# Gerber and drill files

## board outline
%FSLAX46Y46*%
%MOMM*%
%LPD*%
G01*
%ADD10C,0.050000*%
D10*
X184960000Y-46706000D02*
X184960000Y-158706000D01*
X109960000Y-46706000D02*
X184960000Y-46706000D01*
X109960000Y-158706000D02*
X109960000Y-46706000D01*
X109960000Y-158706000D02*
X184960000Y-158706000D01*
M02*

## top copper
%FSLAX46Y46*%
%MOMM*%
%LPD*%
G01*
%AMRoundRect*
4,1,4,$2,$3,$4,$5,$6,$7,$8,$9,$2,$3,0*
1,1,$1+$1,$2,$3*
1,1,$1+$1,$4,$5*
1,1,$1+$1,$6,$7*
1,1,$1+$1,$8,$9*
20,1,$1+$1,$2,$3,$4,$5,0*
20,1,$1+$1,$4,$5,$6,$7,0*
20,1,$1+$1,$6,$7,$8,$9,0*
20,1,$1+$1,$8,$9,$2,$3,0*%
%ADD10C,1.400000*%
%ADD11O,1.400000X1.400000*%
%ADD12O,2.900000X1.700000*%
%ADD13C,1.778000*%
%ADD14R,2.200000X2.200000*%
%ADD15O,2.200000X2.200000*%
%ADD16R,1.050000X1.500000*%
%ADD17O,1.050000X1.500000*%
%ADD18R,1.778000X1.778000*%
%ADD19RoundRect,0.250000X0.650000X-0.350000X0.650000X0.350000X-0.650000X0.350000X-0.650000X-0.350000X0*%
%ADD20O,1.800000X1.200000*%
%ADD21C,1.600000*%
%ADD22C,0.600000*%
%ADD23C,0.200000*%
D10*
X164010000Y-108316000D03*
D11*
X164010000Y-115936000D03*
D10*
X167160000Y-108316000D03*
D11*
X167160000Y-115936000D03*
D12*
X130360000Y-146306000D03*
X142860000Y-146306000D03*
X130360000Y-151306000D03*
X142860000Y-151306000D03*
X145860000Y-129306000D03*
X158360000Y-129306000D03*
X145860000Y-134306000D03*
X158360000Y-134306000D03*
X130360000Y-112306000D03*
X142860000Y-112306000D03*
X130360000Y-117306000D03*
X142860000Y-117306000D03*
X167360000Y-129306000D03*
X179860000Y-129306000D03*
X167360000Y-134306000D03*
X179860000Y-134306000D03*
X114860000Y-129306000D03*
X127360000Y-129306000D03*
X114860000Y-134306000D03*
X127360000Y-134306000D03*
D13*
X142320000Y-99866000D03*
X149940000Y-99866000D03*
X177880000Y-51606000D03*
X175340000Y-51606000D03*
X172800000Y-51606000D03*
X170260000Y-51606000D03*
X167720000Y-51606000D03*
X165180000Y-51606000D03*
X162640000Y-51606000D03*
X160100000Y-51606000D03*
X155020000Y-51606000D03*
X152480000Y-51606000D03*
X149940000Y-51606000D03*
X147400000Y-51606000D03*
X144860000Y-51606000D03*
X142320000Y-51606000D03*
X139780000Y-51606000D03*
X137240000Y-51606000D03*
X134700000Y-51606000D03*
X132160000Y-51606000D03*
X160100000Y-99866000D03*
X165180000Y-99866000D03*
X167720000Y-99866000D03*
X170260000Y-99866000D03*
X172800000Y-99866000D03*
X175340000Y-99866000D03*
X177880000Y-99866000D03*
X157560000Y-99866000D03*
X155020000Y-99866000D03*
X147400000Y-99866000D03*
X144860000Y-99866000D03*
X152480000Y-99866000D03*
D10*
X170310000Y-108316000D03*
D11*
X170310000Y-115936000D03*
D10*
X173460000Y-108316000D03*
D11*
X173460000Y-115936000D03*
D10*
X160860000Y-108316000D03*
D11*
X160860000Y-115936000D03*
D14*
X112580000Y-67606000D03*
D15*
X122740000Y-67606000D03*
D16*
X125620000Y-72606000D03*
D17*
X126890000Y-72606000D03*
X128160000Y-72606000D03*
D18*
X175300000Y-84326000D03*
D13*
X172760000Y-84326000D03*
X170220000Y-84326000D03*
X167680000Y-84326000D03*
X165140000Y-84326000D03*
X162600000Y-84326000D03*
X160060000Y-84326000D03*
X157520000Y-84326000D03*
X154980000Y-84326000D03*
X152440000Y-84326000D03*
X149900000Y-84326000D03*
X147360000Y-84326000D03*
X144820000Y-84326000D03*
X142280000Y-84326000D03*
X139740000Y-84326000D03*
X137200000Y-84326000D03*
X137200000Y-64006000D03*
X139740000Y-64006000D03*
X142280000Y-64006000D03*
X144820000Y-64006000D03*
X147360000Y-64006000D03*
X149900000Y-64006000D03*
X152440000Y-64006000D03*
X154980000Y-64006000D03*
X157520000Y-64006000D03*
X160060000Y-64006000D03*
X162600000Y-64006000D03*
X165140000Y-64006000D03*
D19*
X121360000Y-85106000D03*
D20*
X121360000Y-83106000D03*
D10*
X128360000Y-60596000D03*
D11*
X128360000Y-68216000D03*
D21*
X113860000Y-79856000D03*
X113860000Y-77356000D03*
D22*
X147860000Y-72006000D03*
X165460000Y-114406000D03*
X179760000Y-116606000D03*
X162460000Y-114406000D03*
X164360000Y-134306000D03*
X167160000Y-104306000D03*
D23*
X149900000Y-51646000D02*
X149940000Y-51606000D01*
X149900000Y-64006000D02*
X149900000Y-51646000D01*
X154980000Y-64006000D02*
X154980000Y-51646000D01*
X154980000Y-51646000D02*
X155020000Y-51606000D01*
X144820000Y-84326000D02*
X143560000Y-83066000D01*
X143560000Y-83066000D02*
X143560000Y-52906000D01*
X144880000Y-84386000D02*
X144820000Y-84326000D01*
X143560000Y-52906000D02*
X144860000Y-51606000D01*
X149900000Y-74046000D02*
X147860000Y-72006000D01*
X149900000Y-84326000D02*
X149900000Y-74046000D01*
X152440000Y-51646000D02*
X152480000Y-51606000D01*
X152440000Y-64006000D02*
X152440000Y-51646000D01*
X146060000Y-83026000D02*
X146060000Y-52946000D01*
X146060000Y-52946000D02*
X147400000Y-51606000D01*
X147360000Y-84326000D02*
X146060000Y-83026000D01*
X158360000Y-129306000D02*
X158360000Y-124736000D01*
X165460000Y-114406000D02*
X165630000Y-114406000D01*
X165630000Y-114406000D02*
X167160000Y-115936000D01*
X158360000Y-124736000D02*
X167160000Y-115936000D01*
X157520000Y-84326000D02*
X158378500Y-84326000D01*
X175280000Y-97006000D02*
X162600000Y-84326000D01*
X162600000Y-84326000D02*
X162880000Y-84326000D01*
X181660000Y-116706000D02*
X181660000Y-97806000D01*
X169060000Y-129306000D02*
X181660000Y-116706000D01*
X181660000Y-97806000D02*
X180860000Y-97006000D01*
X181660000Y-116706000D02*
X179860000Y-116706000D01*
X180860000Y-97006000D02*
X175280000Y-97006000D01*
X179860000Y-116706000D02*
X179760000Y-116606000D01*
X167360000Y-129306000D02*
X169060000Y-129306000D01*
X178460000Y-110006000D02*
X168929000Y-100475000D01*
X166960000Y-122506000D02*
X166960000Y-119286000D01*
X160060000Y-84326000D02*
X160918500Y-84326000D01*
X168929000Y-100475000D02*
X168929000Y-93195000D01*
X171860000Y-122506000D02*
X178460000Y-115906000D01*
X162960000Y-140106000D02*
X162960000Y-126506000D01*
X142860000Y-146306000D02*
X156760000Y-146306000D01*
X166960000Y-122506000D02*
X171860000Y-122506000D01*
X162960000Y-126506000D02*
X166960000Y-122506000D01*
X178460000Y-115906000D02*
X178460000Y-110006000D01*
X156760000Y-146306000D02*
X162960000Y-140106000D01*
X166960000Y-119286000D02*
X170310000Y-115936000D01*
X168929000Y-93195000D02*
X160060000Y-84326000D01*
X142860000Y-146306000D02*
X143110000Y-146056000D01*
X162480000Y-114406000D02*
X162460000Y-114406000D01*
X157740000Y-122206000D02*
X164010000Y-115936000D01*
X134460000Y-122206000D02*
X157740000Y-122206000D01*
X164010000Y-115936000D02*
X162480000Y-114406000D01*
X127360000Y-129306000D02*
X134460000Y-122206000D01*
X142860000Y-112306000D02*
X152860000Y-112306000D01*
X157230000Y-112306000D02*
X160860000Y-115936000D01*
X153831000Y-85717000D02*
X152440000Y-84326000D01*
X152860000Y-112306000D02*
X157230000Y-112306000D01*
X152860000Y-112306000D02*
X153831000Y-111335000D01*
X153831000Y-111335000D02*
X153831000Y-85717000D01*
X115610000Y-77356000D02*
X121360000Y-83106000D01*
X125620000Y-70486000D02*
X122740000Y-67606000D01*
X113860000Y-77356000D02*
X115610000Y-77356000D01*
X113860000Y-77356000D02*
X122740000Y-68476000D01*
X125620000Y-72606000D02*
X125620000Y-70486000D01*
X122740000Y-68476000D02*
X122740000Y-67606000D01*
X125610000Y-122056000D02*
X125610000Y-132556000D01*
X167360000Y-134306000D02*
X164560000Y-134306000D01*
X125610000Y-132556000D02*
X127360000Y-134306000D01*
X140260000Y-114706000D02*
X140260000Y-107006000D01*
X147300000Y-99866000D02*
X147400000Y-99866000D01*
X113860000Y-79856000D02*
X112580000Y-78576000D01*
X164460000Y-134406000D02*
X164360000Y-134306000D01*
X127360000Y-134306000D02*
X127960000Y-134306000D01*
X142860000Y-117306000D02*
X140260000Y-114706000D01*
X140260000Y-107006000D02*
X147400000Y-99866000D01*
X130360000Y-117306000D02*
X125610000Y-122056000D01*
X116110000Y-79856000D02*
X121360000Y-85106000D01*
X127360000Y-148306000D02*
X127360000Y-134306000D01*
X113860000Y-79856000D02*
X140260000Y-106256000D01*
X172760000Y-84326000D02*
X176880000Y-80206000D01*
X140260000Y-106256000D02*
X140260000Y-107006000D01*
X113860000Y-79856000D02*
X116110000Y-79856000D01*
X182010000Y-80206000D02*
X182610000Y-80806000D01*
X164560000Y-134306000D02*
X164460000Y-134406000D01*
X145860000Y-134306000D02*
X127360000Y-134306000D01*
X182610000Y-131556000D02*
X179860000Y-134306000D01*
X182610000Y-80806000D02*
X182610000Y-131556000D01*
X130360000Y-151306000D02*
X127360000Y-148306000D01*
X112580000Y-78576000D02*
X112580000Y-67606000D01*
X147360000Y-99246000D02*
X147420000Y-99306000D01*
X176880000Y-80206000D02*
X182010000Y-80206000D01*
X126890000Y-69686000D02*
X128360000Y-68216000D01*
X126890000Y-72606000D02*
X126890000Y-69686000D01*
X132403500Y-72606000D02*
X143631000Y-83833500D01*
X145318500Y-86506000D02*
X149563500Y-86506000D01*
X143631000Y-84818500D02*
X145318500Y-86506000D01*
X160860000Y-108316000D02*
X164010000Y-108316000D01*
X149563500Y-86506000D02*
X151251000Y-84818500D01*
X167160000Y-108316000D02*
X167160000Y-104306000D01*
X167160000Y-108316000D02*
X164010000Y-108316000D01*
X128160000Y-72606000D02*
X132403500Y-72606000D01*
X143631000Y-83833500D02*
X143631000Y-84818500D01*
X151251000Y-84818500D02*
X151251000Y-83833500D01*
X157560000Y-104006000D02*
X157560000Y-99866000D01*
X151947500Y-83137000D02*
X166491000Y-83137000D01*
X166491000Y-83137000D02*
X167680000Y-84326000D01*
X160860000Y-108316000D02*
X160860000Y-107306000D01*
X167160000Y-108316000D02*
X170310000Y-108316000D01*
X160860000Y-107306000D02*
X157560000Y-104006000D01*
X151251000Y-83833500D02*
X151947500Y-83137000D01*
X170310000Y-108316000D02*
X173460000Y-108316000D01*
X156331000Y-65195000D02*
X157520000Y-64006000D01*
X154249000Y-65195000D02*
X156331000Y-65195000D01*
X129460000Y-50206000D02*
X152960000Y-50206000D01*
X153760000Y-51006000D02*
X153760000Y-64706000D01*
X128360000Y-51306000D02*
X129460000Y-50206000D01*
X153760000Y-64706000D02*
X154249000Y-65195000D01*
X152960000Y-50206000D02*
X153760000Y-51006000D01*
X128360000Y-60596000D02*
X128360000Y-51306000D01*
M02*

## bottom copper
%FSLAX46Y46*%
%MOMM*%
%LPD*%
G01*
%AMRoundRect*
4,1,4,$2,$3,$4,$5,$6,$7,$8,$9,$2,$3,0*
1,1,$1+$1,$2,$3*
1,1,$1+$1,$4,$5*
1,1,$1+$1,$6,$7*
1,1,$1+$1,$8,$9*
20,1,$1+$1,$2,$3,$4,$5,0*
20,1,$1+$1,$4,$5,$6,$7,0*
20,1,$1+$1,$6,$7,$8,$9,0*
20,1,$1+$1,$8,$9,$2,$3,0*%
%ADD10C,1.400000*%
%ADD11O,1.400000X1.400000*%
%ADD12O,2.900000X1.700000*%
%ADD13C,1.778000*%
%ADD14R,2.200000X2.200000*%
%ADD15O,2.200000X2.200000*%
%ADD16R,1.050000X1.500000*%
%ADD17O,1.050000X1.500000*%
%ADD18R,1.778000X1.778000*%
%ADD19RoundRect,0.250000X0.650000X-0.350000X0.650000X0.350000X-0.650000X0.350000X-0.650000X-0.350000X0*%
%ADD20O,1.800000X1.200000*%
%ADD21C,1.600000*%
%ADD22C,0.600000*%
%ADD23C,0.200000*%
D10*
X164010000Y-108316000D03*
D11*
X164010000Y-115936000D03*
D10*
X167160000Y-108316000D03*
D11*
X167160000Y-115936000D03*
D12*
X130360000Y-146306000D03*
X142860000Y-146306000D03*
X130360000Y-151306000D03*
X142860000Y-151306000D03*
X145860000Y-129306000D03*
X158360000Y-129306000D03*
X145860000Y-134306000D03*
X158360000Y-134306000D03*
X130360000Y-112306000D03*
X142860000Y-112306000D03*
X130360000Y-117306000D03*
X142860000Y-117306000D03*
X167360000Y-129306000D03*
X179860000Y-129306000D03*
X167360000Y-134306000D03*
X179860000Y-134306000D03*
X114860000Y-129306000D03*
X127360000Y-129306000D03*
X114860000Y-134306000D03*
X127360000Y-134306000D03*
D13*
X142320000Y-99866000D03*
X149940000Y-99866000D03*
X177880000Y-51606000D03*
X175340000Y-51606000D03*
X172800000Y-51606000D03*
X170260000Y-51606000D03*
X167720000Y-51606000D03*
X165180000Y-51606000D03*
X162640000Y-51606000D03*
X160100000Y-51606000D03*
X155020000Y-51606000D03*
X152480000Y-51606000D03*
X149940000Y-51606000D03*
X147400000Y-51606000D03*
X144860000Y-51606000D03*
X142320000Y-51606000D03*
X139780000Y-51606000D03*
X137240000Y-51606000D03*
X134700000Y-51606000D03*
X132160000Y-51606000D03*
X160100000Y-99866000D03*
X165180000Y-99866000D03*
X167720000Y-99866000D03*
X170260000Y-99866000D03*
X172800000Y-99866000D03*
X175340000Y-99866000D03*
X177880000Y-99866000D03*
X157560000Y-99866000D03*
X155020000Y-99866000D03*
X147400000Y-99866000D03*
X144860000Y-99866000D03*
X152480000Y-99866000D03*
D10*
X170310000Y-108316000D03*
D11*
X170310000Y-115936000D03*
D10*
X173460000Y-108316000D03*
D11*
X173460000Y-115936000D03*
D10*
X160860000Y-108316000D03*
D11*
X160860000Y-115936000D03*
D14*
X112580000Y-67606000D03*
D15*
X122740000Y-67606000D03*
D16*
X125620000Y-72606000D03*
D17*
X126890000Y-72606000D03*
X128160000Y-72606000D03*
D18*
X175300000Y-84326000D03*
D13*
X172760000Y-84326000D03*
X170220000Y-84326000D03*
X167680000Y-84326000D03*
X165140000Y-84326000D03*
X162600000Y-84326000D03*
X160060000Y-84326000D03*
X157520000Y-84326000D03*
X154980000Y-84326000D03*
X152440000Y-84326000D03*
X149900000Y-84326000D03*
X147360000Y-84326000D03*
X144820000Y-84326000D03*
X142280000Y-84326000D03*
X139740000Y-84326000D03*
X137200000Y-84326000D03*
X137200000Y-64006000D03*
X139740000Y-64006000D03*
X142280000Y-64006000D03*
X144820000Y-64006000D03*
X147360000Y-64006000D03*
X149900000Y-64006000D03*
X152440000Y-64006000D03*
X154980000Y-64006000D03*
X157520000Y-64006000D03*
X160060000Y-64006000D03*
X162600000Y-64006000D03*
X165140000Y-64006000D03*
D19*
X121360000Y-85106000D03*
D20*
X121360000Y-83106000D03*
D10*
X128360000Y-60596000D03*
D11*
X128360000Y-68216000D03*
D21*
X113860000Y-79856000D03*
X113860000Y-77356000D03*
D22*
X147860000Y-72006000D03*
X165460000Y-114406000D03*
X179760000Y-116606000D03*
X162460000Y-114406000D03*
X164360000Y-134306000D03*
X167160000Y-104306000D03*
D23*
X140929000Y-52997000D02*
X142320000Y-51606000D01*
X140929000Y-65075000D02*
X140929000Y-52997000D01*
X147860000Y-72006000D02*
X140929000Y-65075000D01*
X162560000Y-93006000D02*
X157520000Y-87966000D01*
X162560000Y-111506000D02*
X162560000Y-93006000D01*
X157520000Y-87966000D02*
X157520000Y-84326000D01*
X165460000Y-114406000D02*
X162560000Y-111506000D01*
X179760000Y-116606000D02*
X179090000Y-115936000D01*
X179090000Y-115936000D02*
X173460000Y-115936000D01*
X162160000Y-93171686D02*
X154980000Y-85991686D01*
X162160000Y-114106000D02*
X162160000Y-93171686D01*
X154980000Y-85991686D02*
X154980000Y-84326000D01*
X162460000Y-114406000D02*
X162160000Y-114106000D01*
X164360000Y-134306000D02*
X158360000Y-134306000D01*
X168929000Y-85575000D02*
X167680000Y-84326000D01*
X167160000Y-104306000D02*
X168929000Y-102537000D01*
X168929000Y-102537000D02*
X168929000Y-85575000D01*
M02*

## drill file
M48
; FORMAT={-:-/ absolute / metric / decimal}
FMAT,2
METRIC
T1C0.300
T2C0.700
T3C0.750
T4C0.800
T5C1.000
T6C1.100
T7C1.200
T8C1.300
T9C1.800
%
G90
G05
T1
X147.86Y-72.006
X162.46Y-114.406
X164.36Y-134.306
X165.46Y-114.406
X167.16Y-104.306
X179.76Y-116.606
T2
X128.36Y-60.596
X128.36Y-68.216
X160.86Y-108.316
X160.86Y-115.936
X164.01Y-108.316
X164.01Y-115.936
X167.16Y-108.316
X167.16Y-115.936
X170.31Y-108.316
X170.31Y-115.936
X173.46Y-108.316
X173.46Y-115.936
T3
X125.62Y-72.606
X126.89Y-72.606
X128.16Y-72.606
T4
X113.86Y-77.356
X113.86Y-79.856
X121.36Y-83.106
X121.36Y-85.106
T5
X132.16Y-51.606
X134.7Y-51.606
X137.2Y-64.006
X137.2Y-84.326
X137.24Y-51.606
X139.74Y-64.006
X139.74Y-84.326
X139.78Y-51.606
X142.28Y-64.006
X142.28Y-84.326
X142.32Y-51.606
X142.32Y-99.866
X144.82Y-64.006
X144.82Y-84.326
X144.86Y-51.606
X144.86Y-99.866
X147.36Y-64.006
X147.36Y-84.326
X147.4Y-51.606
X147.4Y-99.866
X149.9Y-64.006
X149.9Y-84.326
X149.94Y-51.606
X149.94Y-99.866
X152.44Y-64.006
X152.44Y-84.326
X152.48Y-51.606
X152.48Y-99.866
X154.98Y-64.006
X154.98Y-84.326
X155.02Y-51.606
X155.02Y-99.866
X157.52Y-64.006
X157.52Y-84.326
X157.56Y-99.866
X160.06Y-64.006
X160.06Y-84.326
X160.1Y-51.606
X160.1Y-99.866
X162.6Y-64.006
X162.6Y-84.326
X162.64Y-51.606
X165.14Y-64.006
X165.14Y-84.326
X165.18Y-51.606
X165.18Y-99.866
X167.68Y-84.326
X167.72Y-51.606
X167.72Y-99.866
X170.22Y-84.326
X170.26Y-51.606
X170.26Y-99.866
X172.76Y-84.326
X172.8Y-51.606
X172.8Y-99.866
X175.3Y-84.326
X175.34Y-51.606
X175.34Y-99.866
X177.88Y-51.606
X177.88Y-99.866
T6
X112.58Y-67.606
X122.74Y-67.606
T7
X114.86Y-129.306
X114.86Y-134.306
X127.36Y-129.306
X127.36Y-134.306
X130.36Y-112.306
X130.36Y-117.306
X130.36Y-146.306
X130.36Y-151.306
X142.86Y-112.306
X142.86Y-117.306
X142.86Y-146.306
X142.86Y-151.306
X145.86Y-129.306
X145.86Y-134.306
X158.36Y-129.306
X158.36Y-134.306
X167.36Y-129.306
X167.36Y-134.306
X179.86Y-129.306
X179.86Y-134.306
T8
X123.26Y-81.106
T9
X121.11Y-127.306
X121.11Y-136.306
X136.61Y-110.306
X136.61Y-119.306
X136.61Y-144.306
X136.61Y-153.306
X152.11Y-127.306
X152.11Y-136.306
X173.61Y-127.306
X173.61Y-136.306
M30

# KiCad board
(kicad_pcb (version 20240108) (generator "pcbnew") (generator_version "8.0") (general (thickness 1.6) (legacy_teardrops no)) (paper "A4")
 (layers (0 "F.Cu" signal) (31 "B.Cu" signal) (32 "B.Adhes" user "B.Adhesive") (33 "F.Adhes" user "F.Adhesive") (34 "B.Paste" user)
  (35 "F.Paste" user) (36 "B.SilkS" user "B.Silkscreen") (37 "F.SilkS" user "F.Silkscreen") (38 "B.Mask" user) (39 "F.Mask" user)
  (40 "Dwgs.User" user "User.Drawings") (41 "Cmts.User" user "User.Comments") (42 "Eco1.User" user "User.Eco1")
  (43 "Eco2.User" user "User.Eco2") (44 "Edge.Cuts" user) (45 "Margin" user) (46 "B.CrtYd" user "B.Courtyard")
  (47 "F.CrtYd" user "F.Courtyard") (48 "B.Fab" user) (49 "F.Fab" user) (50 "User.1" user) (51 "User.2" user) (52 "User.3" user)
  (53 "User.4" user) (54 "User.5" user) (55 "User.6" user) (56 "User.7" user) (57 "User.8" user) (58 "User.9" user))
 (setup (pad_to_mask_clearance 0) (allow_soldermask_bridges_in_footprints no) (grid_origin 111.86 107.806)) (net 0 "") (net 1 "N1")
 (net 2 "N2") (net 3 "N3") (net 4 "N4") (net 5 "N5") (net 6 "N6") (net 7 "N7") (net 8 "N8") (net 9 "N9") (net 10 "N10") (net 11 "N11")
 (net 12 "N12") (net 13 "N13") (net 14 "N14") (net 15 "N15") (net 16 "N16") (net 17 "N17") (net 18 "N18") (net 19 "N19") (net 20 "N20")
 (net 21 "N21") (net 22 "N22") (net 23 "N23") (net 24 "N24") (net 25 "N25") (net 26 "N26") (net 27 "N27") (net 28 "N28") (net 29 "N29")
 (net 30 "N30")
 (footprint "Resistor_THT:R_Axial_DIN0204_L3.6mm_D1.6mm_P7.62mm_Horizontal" (layer "F.Cu") (at 164.01 108.316 -90)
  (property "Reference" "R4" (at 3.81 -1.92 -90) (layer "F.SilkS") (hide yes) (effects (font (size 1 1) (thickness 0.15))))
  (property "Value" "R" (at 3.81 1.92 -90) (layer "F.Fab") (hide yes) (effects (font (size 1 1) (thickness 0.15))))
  (pad "1" thru_hole circle (at 0 0 270) (size 1.4 1.4) (drill 0.7) (layers "*.Cu" "*.Mask") (remove_unused_layers no) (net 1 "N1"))
  (pad "2" thru_hole oval (at 7.62 0 270) (size 1.4 1.4) (drill 0.7) (layers "*.Cu" "*.Mask") (remove_unused_layers no) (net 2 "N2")))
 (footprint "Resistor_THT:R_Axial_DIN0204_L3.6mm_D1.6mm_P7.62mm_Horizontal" (layer "F.Cu") (at 167.16 108.316 -90)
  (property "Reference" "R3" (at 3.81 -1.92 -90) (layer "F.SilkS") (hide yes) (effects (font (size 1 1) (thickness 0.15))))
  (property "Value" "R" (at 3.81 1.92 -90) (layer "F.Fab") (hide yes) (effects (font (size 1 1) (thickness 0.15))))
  (pad "1" thru_hole circle (at 0 0 270) (size 1.4 1.4) (drill 0.7) (layers "*.Cu" "*.Mask") (remove_unused_layers no) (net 1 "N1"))
  (pad "2" thru_hole oval (at 7.62 0 270) (size 1.4 1.4) (drill 0.7) (layers "*.Cu" "*.Mask") (remove_unused_layers no) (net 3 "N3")))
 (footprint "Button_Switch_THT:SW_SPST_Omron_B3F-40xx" (layer "F.Cu") (at 130.36 146.306)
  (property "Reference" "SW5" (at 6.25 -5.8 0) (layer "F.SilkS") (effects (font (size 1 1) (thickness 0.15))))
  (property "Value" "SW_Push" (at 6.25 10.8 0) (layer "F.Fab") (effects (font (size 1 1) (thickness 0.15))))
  (pad "" np_thru_hole circle (at 6.25 -2) (size 1.8 1.8) (drill 1.8) (layers "F&B.Cu" "*.Mask"))
  (pad "" np_thru_hole circle (at 6.25 7) (size 1.8 1.8) (drill 1.8) (layers "F&B.Cu" "*.Mask"))
  (pad "1" thru_hole oval (at 0 0) (size 2.9 1.7) (drill 1.2) (layers "*.Cu" "*.Mask") (remove_unused_layers no) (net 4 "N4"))
  (pad "1" thru_hole oval (at 12.5 0) (size 2.9 1.7) (drill 1.2) (layers "*.Cu" "*.Mask") (remove_unused_layers no) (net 4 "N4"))
  (pad "2" thru_hole oval (at 0 5) (size 2.9 1.7) (drill 1.2) (layers "*.Cu" "*.Mask") (remove_unused_layers no) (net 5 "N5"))
  (pad "2" thru_hole oval (at 12.5 5) (size 2.9 1.7) (drill 1.2) (layers "*.Cu" "*.Mask") (remove_unused_layers no) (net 5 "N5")))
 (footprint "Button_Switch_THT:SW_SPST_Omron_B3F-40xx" (layer "F.Cu") (at 145.86 129.306)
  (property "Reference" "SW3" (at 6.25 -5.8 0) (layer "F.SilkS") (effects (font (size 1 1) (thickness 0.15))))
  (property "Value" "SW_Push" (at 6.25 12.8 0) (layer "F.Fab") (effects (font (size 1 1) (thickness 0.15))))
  (pad "" np_thru_hole circle (at 6.25 -2) (size 1.8 1.8) (drill 1.8) (layers "F&B.Cu" "*.Mask"))
  (pad "" np_thru_hole circle (at 6.25 7) (size 1.8 1.8) (drill 1.8) (layers "F&B.Cu" "*.Mask"))
  (pad "1" thru_hole oval (at 0 0) (size 2.9 1.7) (drill 1.2) (layers "*.Cu" "*.Mask") (remove_unused_layers no) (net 3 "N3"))
  (pad "1" thru_hole oval (at 12.5 0) (size 2.9 1.7) (drill 1.2) (layers "*.Cu" "*.Mask") (remove_unused_layers no) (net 3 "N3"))
  (pad "2" thru_hole oval (at 0 5) (size 2.9 1.7) (drill 1.2) (layers "*.Cu" "*.Mask") (remove_unused_layers no) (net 5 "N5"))
  (pad "2" thru_hole oval (at 12.5 5) (size 2.9 1.7) (drill 1.2) (layers "*.Cu" "*.Mask") (remove_unused_layers no) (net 5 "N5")))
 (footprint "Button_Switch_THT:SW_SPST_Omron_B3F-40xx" (layer "F.Cu") (at 130.36 112.306)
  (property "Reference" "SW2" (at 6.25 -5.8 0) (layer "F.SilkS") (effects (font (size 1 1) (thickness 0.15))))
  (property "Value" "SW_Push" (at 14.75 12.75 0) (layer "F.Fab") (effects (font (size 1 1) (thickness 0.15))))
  (pad "" np_thru_hole circle (at 6.25 -2) (size 1.8 1.8) (drill 1.8) (layers "F&B.Cu" "*.Mask"))
  (pad "" np_thru_hole circle (at 6.25 7) (size 1.8 1.8) (drill 1.8) (layers "F&B.Cu" "*.Mask"))
  (pad "1" thru_hole oval (at 0 0) (size 2.9 1.7) (drill 1.2) (layers "*.Cu" "*.Mask") (remove_unused_layers no) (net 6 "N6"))
  (pad "1" thru_hole oval (at 12.5 0) (size 2.9 1.7) (drill 1.2) (layers "*.Cu" "*.Mask") (remove_unused_layers no) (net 6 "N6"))
  (pad "2" thru_hole oval (at 0 5) (size 2.9 1.7) (drill 1.2) (layers "*.Cu" "*.Mask") (remove_unused_layers no) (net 5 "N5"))
  (pad "2" thru_hole oval (at 12.5 5) (size 2.9 1.7) (drill 1.2) (layers "*.Cu" "*.Mask") (remove_unused_layers no) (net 5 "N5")))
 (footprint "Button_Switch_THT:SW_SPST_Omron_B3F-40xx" (layer "F.Cu") (at 167.36 129.306)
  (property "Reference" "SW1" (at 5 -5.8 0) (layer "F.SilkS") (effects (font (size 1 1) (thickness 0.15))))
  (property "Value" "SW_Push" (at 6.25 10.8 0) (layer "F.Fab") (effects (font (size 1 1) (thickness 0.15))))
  (pad "" np_thru_hole circle (at 6.25 -2) (size 1.8 1.8) (drill 1.8) (layers "F&B.Cu" "*.Mask"))
  (pad "" np_thru_hole circle (at 6.25 7) (size 1.8 1.8) (drill 1.8) (layers "F&B.Cu" "*.Mask"))
  (pad "1" thru_hole oval (at 0 0) (size 2.9 1.7) (drill 1.2) (layers "*.Cu" "*.Mask") (remove_unused_layers no) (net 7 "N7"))
  (pad "1" thru_hole oval (at 12.5 0) (size 2.9 1.7) (drill 1.2) (layers "*.Cu" "*.Mask") (remove_unused_layers no) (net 7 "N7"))
  (pad "2" thru_hole oval (at 0 5) (size 2.9 1.7) (drill 1.2) (layers "*.Cu" "*.Mask") (remove_unused_layers no) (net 5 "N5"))
  (pad "2" thru_hole oval (at 12.5 5) (size 2.9 1.7) (drill 1.2) (layers "*.Cu" "*.Mask") (remove_unused_layers no) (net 5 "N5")))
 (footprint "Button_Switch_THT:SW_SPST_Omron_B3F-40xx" (layer "F.Cu") (at 114.86 129.306)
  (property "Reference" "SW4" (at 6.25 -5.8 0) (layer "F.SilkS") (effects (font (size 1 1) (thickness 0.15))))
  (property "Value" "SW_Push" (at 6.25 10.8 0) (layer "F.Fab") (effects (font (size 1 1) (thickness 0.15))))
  (pad "" np_thru_hole circle (at 6.25 -2) (size 1.8 1.8) (drill 1.8) (layers "F&B.Cu" "*.Mask"))
  (pad "" np_thru_hole circle (at 6.25 7) (size 1.8 1.8) (drill 1.8) (layers "F&B.Cu" "*.Mask"))
  (pad "1" thru_hole oval (at 0 0) (size 2.9 1.7) (drill 1.2) (layers "*.Cu" "*.Mask") (remove_unused_layers no) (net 2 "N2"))
  (pad "1" thru_hole oval (at 12.5 0) (size 2.9 1.7) (drill 1.2) (layers "*.Cu" "*.Mask") (remove_unused_layers no) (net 2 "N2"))
  (pad "2" thru_hole oval (at 0 5) (size 2.9 1.7) (drill 1.2) (layers "*.Cu" "*.Mask") (remove_unused_layers no) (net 5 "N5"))
  (pad "2" thru_hole oval (at 12.5 5) (size 2.9 1.7) (drill 1.2) (layers "*.Cu" "*.Mask") (remove_unused_layers no) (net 5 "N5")))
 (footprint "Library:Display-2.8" (layer "F.Cu") (at 177.88 51.606 90)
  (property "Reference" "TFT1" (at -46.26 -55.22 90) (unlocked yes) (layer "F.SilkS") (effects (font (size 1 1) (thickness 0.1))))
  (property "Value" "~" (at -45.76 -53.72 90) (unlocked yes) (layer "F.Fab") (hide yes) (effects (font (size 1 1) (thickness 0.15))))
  (pad "" thru_hole circle (at -48.26 -35.56 90) (size 1.778 1.778) (drill 1) (layers "*.Cu" "*.Mask") (remove_unused_layers no))
  (pad "" thru_hole circle (at -48.26 -27.94 90) (size 1.778 1.778) (drill 1) (layers "*.Cu" "*.Mask") (remove_unused_layers no))
  (pad "0" thru_hole circle (at 0 0 90) (size 1.778 1.778) (drill 1) (layers "*.Cu" "*.Mask") (remove_unused_layers no))
  (pad "1" thru_hole circle (at 0 -2.54 90) (size 1.778 1.778) (drill 1) (layers "*.Cu" "*.Mask") (remove_unused_layers no))
  (pad "2" thru_hole circle (at 0 -5.08 90) (size 1.778 1.778) (drill 1) (layers "*.Cu" "*.Mask") (remove_unused_layers no))
  (pad "3" thru_hole circle (at 0 -7.62 90) (size 1.778 1.778) (drill 1) (layers "*.Cu" "*.Mask") (remove_unused_layers no))
  (pad "4" thru_hole circle (at 0 -10.16 90) (size 1.778 1.778) (drill 1) (layers "*.Cu" "*.Mask") (remove_unused_layers no) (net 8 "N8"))
  (pad "5" thru_hole circle (at 0 -12.7 90) (size 1.778 1.778) (drill 1) (layers "*.Cu" "*.Mask") (remove_unused_layers no))
  (pad "6" thru_hole circle (at 0 -15.24 90) (size 1.778 1.778) (drill 1) (layers "*.Cu" "*.Mask") (remove_unused_layers no))
  (pad "7" thru_hole circle (at 0 -17.78 90) (size 1.778 1.778) (drill 1) (layers "*.Cu" "*.Mask") (remove_unused_layers no))
  (pad "8" thru_hole circle (at 0 -22.86 90) (size 1.778 1.778) (drill 1) (layers "*.Cu" "*.Mask") (remove_unused_layers no) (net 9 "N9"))
  (pad "9" thru_hole circle (at 0 -25.4 90) (size 1.778 1.778) (drill 1) (layers "*.Cu" "*.Mask") (remove_unused_layers no) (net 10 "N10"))
  (pad "10" thru_hole circle (at 0 -27.94 90) (size 1.778 1.778) (drill 1) (layers "*.Cu" "*.Mask") (remove_unused_layers no) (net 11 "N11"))
  (pad "11" thru_hole circle (at 0 -30.48 90) (size 1.778 1.778) (drill 1) (layers "*.Cu" "*.Mask") (remove_unused_layers no) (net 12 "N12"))
  (pad "12" thru_hole circle (at 0 -33.02 90) (size 1.778 1.778) (drill 1) (layers "*.Cu" "*.Mask") (remove_unused_layers no) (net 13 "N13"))
  (pad "13" thru_hole circle (at 0 -35.56 90) (size 1.778 1.778) (drill 1) (layers "*.Cu" "*.Mask" "Dwgs.User") (remove_unused_layers no)
   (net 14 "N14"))
  (pad "14" thru_hole circle (at 0 -38.1 90) (size 1.778 1.778) (drill 1) (layers "*.Cu" "B.Mask") (remove_unused_layers no))
  (pad "15" thru_hole circle (at 0 -40.64 90) (size 1.778 1.778) (drill 1) (layers "*.Cu" "*.Mask" "B.SilkS") (remove_unused_layers no))
  (pad "16" thru_hole circle (at 0 -43.18 90) (size 1.778 1.778) (drill 1) (layers "*.Cu" "*.Mask") (remove_unused_layers no))
  (pad "17" thru_hole circle (at 0 -45.72 90) (size 1.778 1.778) (drill 1) (layers "*.Cu" "*.Mask" "F.Paste") (remove_unused_layers no))
  (pad "22" thru_hole circle (at -48.26 -17.78 90) (size 1.778 1.778) (drill 1) (layers "*.Cu" "*.Mask") (remove_unused_layers no))
  (pad "23" thru_hole circle (at -48.26 -12.7 90) (size 1.778 1.778) (drill 1) (layers "*.Cu" "*.Mask") (remove_unused_layers no))
  (pad "24" thru_hole circle (at -48.26 -10.16 90) (size 1.778 1.778) (drill 1) (layers "*.Cu" "*.Mask") (remove_unused_layers no))
  (pad "25" thru_hole circle (at -48.26 -7.62 90) (size 1.778 1.778) (drill 1) (layers "*.Cu" "*.Mask") (remove_unused_layers no))
  (pad "26" thru_hole circle (at -48.26 -5.08 90) (size 1.778 1.778) (drill 1) (layers "*.Cu" "*.Mask") (remove_unused_layers no))
  (pad "27" thru_hole circle (at -48.26 -2.54 90) (size 1.778 1.778) (drill 1) (layers "*.Cu" "*.Mask") (remove_unused_layers no))
  (pad "28" thru_hole circle (at -48.26 0 90) (size 1.778 1.778) (drill 1) (layers "*.Cu" "*.Mask") (remove_unused_layers no))
  (pad "40" thru_hole circle (at -48.26 -20.32 90) (size 1.778 1.778) (drill 1) (layers "*.Cu" "*.Mask") (remove_unused_layers no)
   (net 1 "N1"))
  (pad "41" thru_hole circle (at -48.26 -22.86 90) (size 1.778 1.778) (drill 1) (layers "*.Cu" "*.Mask") (remove_unused_layers no))
  (pad "50" thru_hole circle (at -48.26 -30.48 90) (size 1.778 1.778) (drill 1) (layers "*.Cu" "*.Mask") (remove_unused_layers no)
   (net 5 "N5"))
  (pad "51" thru_hole circle (at -48.26 -33.02 90) (size 1.778 1.778) (drill 1) (layers "*.Cu" "*.Mask") (remove_unused_layers no))
  (pad "67" thru_hole circle (at -48.26 -25.4 90) (size 1.778 1.778) (drill 1) (layers "*.Cu" "*.Mask") (remove_unused_layers no)))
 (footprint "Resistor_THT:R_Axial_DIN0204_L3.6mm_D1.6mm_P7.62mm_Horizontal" (layer "F.Cu") (at 170.31 108.316 -90)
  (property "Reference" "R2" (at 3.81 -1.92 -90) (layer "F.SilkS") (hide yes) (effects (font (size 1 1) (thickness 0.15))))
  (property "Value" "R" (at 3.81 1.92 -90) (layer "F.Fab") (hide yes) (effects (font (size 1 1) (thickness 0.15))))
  (pad "1" thru_hole circle (at 0 0 270) (size 1.4 1.4) (drill 0.7) (layers "*.Cu" "*.Mask") (remove_unused_layers no) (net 1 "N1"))
  (pad "2" thru_hole oval (at 7.62 0 270) (size 1.4 1.4) (drill 0.7) (layers "*.Cu" "*.Mask") (remove_unused_layers no) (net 4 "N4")))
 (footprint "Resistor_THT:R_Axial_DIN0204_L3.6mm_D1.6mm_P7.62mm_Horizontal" (layer "F.Cu") (at 173.46 108.316 -90)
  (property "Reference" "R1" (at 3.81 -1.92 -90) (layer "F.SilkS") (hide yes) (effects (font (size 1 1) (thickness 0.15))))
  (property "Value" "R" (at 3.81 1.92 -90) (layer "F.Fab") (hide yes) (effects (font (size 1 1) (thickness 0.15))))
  (pad "1" thru_hole circle (at 0 0 270) (size 1.4 1.4) (drill 0.7) (layers "*.Cu" "*.Mask") (remove_unused_layers no) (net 1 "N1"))
  (pad "2" thru_hole oval (at 7.62 0 270) (size 1.4 1.4) (drill 0.7) (layers "*.Cu" "*.Mask") (remove_unused_layers no) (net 7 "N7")))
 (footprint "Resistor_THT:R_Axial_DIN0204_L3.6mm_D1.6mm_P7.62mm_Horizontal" (layer "F.Cu") (at 160.86 108.316 -90)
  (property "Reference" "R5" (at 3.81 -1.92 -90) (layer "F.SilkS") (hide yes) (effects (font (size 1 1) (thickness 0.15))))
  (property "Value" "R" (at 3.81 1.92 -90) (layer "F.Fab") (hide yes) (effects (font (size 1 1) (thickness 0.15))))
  (pad "1" thru_hole circle (at 0 0 270) (size 1.4 1.4) (drill 0.7) (layers "*.Cu" "*.Mask") (remove_unused_layers no) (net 1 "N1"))
  (pad "2" thru_hole oval (at 7.62 0 270) (size 1.4 1.4) (drill 0.7) (layers "*.Cu" "*.Mask") (remove_unused_layers no) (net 6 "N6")))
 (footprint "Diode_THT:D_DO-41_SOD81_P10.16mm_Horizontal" (layer "B.Cu") (at 112.58 67.606)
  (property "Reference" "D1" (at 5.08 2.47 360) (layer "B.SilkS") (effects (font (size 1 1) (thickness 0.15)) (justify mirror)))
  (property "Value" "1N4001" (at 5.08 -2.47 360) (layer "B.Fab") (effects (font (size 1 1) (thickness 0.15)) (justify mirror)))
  (pad "1" thru_hole rect (at 0 0) (size 2.2 2.2) (drill 1.1) (layers "*.Cu" "*.Mask") (remove_unused_layers no) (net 5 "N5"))
  (pad "2" thru_hole oval (at 10.16 0) (size 2.2 2.2) (drill 1.1) (layers "*.Cu" "*.Mask") (remove_unused_layers no) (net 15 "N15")))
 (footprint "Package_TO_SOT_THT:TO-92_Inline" (layer "B.Cu") (at 125.62 72.606)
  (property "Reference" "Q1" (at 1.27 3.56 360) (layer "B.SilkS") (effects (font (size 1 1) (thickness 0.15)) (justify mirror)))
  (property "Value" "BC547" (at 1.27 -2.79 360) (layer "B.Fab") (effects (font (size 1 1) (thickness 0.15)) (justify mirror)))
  (pad "1" thru_hole rect (at 0 0) (size 1.05 1.5) (drill 0.75) (layers "*.Cu" "*.Mask") (remove_unused_layers no) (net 15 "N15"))
  (pad "2" thru_hole oval (at 1.27 0) (size 1.05 1.5) (drill 0.75) (layers "*.Cu" "*.Mask") (remove_unused_layers no) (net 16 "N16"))
  (pad "3" thru_hole oval (at 2.54 0) (size 1.05 1.5) (drill 0.75) (layers "*.Cu" "*.Mask") (remove_unused_layers no) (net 1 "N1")))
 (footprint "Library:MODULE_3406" (layer "B.Cu") (at 156.25 74.166 90)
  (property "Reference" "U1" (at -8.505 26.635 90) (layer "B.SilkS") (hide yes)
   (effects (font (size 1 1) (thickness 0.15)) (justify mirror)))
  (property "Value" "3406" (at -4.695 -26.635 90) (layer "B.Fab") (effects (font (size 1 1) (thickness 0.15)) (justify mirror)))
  (pad "1" thru_hole rect (at -10.16 19.05 90) (size 1.778 1.778) (drill 1) (layers "*.Cu" "*.Mask") (remove_unused_layers no)
   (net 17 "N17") (solder_mask_margin 0.102))
  (pad "2" thru_hole circle (at -10.16 16.51 90) (size 1.778 1.778) (drill 1) (layers "*.Cu" "*.Mask") (remove_unused_layers no)
   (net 5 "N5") (solder_mask_margin 0.102))
  (pad "3" thru_hole circle (at -10.16 13.97 90) (size 1.778 1.778) (drill 1) (layers "*.Cu" "*.Mask") (remove_unused_layers no)
   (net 5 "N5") (solder_mask_margin 0.102))
  (pad "4" thru_hole circle (at -10.16 11.43 90) (size 1.778 1.778) (drill 1) (layers "*.Cu" "*.Mask") (remove_unused_layers no)
   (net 1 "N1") (solder_mask_margin 0.102))
  (pad "5" thru_hole circle (at -10.16 8.89 90) (size 1.778 1.778) (drill 1) (layers "*.Cu" "*.Mask") (remove_unused_layers no)
   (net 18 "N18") (solder_mask_margin 0.102))
  (pad "6" thru_hole circle (at -10.16 6.35 90) (size 1.778 1.778) (drill 1) (layers "*.Cu" "*.Mask") (remove_unused_layers no) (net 7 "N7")
   (solder_mask_margin 0.102))
  (pad "7" thru_hole circle (at -10.16 3.81 90) (size 1.778 1.778) (drill 1) (layers "*.Cu" "*.Mask") (remove_unused_layers no) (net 4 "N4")
   (solder_mask_margin 0.102))
  (pad "8" thru_hole circle (at -10.16 1.27 90) (size 1.778 1.778) (drill 1) (layers "*.Cu" "*.Mask") (remove_unused_layers no) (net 3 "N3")
   (solder_mask_margin 0.102))
  (pad "9" thru_hole circle (at -10.16 -1.27 90) (size 1.778 1.778) (drill 1) (layers "*.Cu" "*.Mask") (remove_unused_layers no)
   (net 2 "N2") (solder_mask_margin 0.102))
  (pad "10" thru_hole circle (at -10.16 -3.81 90) (size 1.778 1.778) (drill 1) (layers "*.Cu" "*.Mask") (remove_unused_layers no)
   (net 6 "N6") (solder_mask_margin 0.102))
  (pad "11" thru_hole circle (at -10.16 -6.35 90) (size 1.778 1.778) (drill 1) (layers "*.Cu" "*.Mask") (remove_unused_layers no)
   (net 14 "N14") (solder_mask_margin 0.102))
  (pad "12" thru_hole circle (at -10.16 -8.89 90) (size 1.778 1.778) (drill 1) (layers "*.Cu" "*.Mask") (remove_unused_layers no)
   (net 12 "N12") (solder_mask_margin 0.102))
  (pad "13" thru_hole circle (at -10.16 -11.43 90) (size 1.778 1.778) (drill 1) (layers "*.Cu" "*.Mask") (remove_unused_layers no)
   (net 13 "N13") (solder_mask_margin 0.102))
  (pad "14" thru_hole circle (at -10.16 -13.97 90) (size 1.778 1.778) (drill 1) (layers "*.Cu" "*.Mask") (remove_unused_layers no)
   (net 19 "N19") (solder_mask_margin 0.102))
  (pad "15" thru_hole circle (at -10.16 -16.51 90) (size 1.778 1.778) (drill 1) (layers "*.Cu" "*.Mask") (remove_unused_layers no)
   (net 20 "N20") (solder_mask_margin 0.102))
  (pad "16" thru_hole circle (at -10.16 -19.05 90) (size 1.778 1.778) (drill 1) (layers "*.Cu" "*.Mask") (remove_unused_layers no)
   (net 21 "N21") (solder_mask_margin 0.102))
  (pad "17" thru_hole circle (at 10.16 -19.05 90) (size 1.778 1.778) (drill 1) (layers "*.Cu" "*.Mask") (remove_unused_layers no)
   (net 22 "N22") (solder_mask_margin 0.102))
  (pad "18" thru_hole circle (at 10.16 -16.51 90) (size 1.778 1.778) (drill 1) (layers "*.Cu" "*.Mask") (remove_unused_layers no)
   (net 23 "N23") (solder_mask_margin 0.102))
  (pad "19" thru_hole circle (at 10.16 -13.97 90) (size 1.778 1.778) (drill 1) (layers "*.Cu" "*.Mask") (remove_unused_layers no)
   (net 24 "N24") (solder_mask_margin 0.102))
  (pad "20" thru_hole circle (at 10.16 -11.43 90) (size 1.778 1.778) (drill 1) (layers "*.Cu" "*.Mask") (remove_unused_layers no)
   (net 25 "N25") (solder_mask_margin 0.102))
  (pad "21" thru_hole circle (at 10.16 -8.89 90) (size 1.778 1.778) (drill 1) (layers "*.Cu" "*.Mask") (remove_unused_layers no)
   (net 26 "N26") (solder_mask_margin 0.102))
  (pad "22" thru_hole circle (at 10.16 -6.35 90) (size 1.778 1.778) (drill 1) (layers "*.Cu" "*.Mask") (remove_unused_layers no)
   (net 11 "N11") (solder_mask_margin 0.102))
  (pad "23" thru_hole circle (at 10.16 -3.81 90) (size 1.778 1.778) (drill 1) (layers "*.Cu" "*.Mask") (remove_unused_layers no)
   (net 10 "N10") (solder_mask_margin 0.102))
  (pad "24" thru_hole circle (at 10.16 -1.27 90) (size 1.778 1.778) (drill 1) (layers "*.Cu" "*.Mask") (remove_unused_layers no)
   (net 9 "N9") (solder_mask_margin 0.102))
  (pad "25" thru_hole circle (at 10.16 1.27 90) (size 1.778 1.778) (drill 1) (layers "*.Cu" "*.Mask") (remove_unused_layers no)
   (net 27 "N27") (solder_mask_margin 0.102))
  (pad "26" thru_hole circle (at 10.16 3.81 90) (size 1.778 1.778) (drill 1) (layers "*.Cu" "*.Mask") (remove_unused_layers no)
   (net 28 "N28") (solder_mask_margin 0.102))
  (pad "27" thru_hole circle (at 10.16 6.35 90) (size 1.778 1.778) (drill 1) (layers "*.Cu" "*.Mask") (remove_unused_layers no)
   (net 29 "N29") (solder_mask_margin 0.102))
  (pad "28" thru_hole circle (at 10.16 8.89 90) (size 1.778 1.778) (drill 1) (layers "*.Cu" "*.Mask") (remove_unused_layers no)
   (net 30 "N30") (solder_mask_margin 0.102)))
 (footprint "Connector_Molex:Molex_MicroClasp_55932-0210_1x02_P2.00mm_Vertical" (layer "B.Cu") (at 121.36 85.106 90)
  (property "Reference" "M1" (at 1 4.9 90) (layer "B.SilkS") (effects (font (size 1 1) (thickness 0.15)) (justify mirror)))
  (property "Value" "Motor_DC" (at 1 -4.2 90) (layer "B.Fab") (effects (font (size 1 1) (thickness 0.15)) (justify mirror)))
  (pad "" np_thru_hole circle (at 4 1.9 90) (size 1.3 1.3) (drill 1.3) (layers "*.Cu" "*.Mask"))
  (pad "1" thru_hole roundrect (at 0 0 90) (size 1.2 1.8) (drill 0.8) (layers "*.Cu" "*.Mask") (remove_unused_layers no)
   (roundrect_rratio 0.208333) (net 5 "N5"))
  (pad "2" thru_hole oval (at 2 0 90) (size 1.2 1.8) (drill 0.8) (layers "*.Cu" "*.Mask") (remove_unused_layers no) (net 15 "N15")))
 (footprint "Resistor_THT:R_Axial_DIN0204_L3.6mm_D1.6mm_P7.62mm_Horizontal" (layer "B.Cu") (at 128.36 60.596 -90)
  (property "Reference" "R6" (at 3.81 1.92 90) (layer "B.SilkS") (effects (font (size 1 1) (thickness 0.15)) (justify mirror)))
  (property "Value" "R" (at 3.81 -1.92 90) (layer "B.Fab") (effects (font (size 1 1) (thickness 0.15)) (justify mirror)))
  (pad "1" thru_hole circle (at 0 0 270) (size 1.4 1.4) (drill 0.7) (layers "*.Cu" "*.Mask") (remove_unused_layers no) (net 27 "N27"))
  (pad "2" thru_hole oval (at 7.62 0 270) (size 1.4 1.4) (drill 0.7) (layers "*.Cu" "*.Mask") (remove_unused_layers no) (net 16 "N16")))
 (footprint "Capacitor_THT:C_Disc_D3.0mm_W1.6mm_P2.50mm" (layer "B.Cu") (at 113.86 79.856 90)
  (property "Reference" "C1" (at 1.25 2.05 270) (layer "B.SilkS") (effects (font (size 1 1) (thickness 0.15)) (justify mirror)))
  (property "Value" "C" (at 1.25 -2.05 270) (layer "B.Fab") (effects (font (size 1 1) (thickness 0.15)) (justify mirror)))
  (pad "1" thru_hole circle (at 0 0 90) (size 1.6 1.6) (drill 0.8) (layers "*.Cu" "*.Mask") (remove_unused_layers no) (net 5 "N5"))
  (pad "2" thru_hole circle (at 2.5 0 90) (size 1.6 1.6) (drill 0.8) (layers "*.Cu" "*.Mask") (remove_unused_layers no) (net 15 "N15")))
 (gr_line (start 184.96 46.706) (end 184.96 158.706) (stroke (width 0.05) (type default)) (layer "Edge.Cuts"))
 (gr_line (start 109.96 46.706) (end 184.96 46.706) (stroke (width 0.05) (type default)) (layer "Edge.Cuts"))
 (gr_line (start 109.96 158.706) (end 109.96 46.706) (stroke (width 0.05) (type default)) (layer "Edge.Cuts"))
 (gr_line (start 109.96 158.706) (end 184.96 158.706) (stroke (width 0.05) (type default)) (layer "Edge.Cuts"))
 (segment (start 149.9 51.646) (end 149.94 51.606) (width 0.2) (layer "F.Cu") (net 11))
 (segment (start 149.9 64.006) (end 149.9 51.646) (width 0.2) (layer "F.Cu") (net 11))
 (segment (start 154.98 64.006) (end 154.98 51.646) (width 0.2) (layer "F.Cu") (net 9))
 (segment (start 154.98 51.646) (end 155.02 51.606) (width 0.2) (layer "F.Cu") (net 9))
 (segment (start 144.82 84.326) (end 143.56 83.066) (width 0.2) (layer "F.Cu") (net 13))
 (segment (start 143.56 83.066) (end 143.56 52.906) (width 0.2) (layer "F.Cu") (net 13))
 (segment (start 144.88 84.386) (end 144.82 84.326) (width 0.2) (layer "F.Cu") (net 13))
 (segment (start 143.56 52.906) (end 144.86 51.606) (width 0.2) (layer "F.Cu") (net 13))
 (segment (start 149.9 74.046) (end 147.86 72.006) (width 0.2) (layer "F.Cu") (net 14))
 (segment (start 149.9 84.326) (end 149.9 74.046) (width 0.2) (layer "F.Cu") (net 14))
 (via (at 147.86 72.006) (size 0.6) (drill 0.3) (layers "F.Cu" "B.Cu") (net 14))
 (segment (start 140.929 52.997) (end 142.32 51.606) (width 0.2) (layer "B.Cu") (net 14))
 (segment (start 140.929 65.075) (end 140.929 52.997) (width 0.2) (layer "B.Cu") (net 14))
 (segment (start 147.86 72.006) (end 140.929 65.075) (width 0.2) (layer "B.Cu") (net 14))
 (segment (start 152.44 51.646) (end 152.48 51.606) (width 0.2) (layer "F.Cu") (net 10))
 (segment (start 152.44 64.006) (end 152.44 51.646) (width 0.2) (layer "F.Cu") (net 10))
 (segment (start 146.06 83.026) (end 146.06 52.946) (width 0.2) (layer "F.Cu") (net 12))
 (segment (start 146.06 52.946) (end 147.4 51.606) (width 0.2) (layer "F.Cu") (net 12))
 (segment (start 147.36 84.326) (end 146.06 83.026) (width 0.2) (layer "F.Cu") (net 12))
 (segment (start 158.36 129.306) (end 158.36 124.736) (width 0.2) (layer "F.Cu") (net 3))
 (segment (start 165.46 114.406) (end 165.63 114.406) (width 0.2) (layer "F.Cu") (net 3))
 (segment (start 165.63 114.406) (end 167.16 115.936) (width 0.2) (layer "F.Cu") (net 3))
 (segment (start 158.36 124.736) (end 167.16 115.936) (width 0.2) (layer "F.Cu") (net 3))
 (segment (start 157.52 84.326) (end 158.3785 84.326) (width 0.2) (layer "F.Cu") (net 3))
 (via (at 165.46 114.406) (size 0.6) (drill 0.3) (layers "F.Cu" "B.Cu") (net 3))
 (segment (start 162.56 93.006) (end 157.52 87.966) (width 0.2) (layer "B.Cu") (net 3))
 (segment (start 162.56 111.506) (end 162.56 93.006) (width 0.2) (layer "B.Cu") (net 3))
 (segment (start 157.52 87.966) (end 157.52 84.326) (width 0.2) (layer "B.Cu") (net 3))
 (segment (start 165.46 114.406) (end 162.56 111.506) (width 0.2) (layer "B.Cu") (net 3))
 (segment (start 175.28 97.006) (end 162.6 84.326) (width 0.2) (layer "F.Cu") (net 7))
 (segment (start 162.6 84.326) (end 162.88 84.326) (width 0.2) (layer "F.Cu") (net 7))
 (segment (start 181.66 116.706) (end 181.66 97.806) (width 0.2) (layer "F.Cu") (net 7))
 (segment (start 169.06 129.306) (end 181.66 116.706) (width 0.2) (layer "F.Cu") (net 7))
 (segment (start 181.66 97.806) (end 180.86 97.006) (width 0.2) (layer "F.Cu") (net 7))
 (segment (start 181.66 116.706) (end 179.86 116.706) (width 0.2) (layer "F.Cu") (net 7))
 (segment (start 180.86 97.006) (end 175.28 97.006) (width 0.2) (layer "F.Cu") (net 7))
 (segment (start 179.86 116.706) (end 179.76 116.606) (width 0.2) (layer "F.Cu") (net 7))
 (segment (start 167.36 129.306) (end 169.06 129.306) (width 0.2) (layer "F.Cu") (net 7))
 (via (at 179.76 116.606) (size 0.6) (drill 0.3) (layers "F.Cu" "B.Cu") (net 7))
 (segment (start 179.76 116.606) (end 179.09 115.936) (width 0.2) (layer "B.Cu") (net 7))
 (segment (start 179.09 115.936) (end 173.46 115.936) (width 0.2) (layer "B.Cu") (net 7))
 (segment (start 178.46 110.006) (end 168.929 100.475) (width 0.2) (layer "F.Cu") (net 4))
 (segment (start 166.96 122.506) (end 166.96 119.286) (width 0.2) (layer "F.Cu") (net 4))
 (segment (start 160.06 84.326) (end 160.9185 84.326) (width 0.2) (layer "F.Cu") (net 4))
 (segment (start 168.929 100.475) (end 168.929 93.195) (width 0.2) (layer "F.Cu") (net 4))
 (segment (start 171.86 122.506) (end 178.46 115.906) (width 0.2) (layer "F.Cu") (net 4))
 (segment (start 162.96 140.106) (end 162.96 126.506) (width 0.2) (layer "F.Cu") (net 4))
 (segment (start 142.86 146.306) (end 156.76 146.306) (width 0.2) (layer "F.Cu") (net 4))
 (segment (start 166.96 122.506) (end 171.86 122.506) (width 0.2) (layer "F.Cu") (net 4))
 (segment (start 162.96 126.506) (end 166.96 122.506) (width 0.2) (layer "F.Cu") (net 4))
 (segment (start 178.46 115.906) (end 178.46 110.006) (width 0.2) (layer "F.Cu") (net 4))
 (segment (start 156.76 146.306) (end 162.96 140.106) (width 0.2) (layer "F.Cu") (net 4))
 (segment (start 166.96 119.286) (end 170.31 115.936) (width 0.2) (layer "F.Cu") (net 4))
 (segment (start 168.929 93.195) (end 160.06 84.326) (width 0.2) (layer "F.Cu") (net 4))
 (segment (start 142.86 146.306) (end 143.11 146.056) (width 0.2) (layer "F.Cu") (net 4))
 (segment (start 162.48 114.406) (end 162.46 114.406) (width 0.2) (layer "F.Cu") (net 2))
 (segment (start 157.74 122.206) (end 164.01 115.936) (width 0.2) (layer "F.Cu") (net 2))
 (segment (start 134.46 122.206) (end 157.74 122.206) (width 0.2) (layer "F.Cu") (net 2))
 (segment (start 164.01 115.936) (end 162.48 114.406) (width 0.2) (layer "F.Cu") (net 2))
 (segment (start 127.36 129.306) (end 134.46 122.206) (width 0.2) (layer "F.Cu") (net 2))
 (via (at 162.46 114.406) (size 0.6) (drill 0.3) (layers "F.Cu" "B.Cu") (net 2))
 (segment (start 162.16 93.171686) (end 154.98 85.991686) (width 0.2) (layer "B.Cu") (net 2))
 (segment (start 162.16 114.106) (end 162.16 93.171686) (width 0.2) (layer "B.Cu") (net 2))
 (segment (start 154.98 85.991686) (end 154.98 84.326) (width 0.2) (layer "B.Cu") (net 2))
 (segment (start 162.46 114.406) (end 162.16 114.106) (width 0.2) (layer "B.Cu") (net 2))
 (segment (start 142.86 112.306) (end 152.86 112.306) (width 0.2) (layer "F.Cu") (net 6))
 (segment (start 157.23 112.306) (end 160.86 115.936) (width 0.2) (layer "F.Cu") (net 6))
 (segment (start 153.831 85.717) (end 152.44 84.326) (width 0.2) (layer "F.Cu") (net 6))
 (segment (start 152.86 112.306) (end 157.23 112.306) (width 0.2) (layer "F.Cu") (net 6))
 (segment (start 152.86 112.306) (end 153.831 111.335) (width 0.2) (layer "F.Cu") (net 6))
 (segment (start 153.831 111.335) (end 153.831 85.717) (width 0.2) (layer "F.Cu") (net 6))
 (segment (start 115.61 77.356) (end 121.36 83.106) (width 0.2) (layer "F.Cu") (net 15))
 (segment (start 125.62 70.486) (end 122.74 67.606) (width 0.2) (layer "F.Cu") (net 15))
 (segment (start 113.86 77.356) (end 115.61 77.356) (width 0.2) (layer "F.Cu") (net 15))
 (segment (start 113.86 77.356) (end 122.74 68.476) (width 0.2) (layer "F.Cu") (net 15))
 (segment (start 125.62 72.606) (end 125.62 70.486) (width 0.2) (layer "F.Cu") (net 15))
 (segment (start 122.74 68.476) (end 122.74 67.606) (width 0.2) (layer "F.Cu") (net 15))
 (segment (start 125.61 122.056) (end 125.61 132.556) (width 0.2) (layer "F.Cu") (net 5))
 (segment (start 167.36 134.306) (end 164.56 134.306) (width 0.2) (layer "F.Cu") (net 5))
 (segment (start 125.61 132.556) (end 127.36 134.306) (width 0.2) (layer "F.Cu") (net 5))
 (segment (start 140.26 114.706) (end 140.26 107.006) (width 0.2) (layer "F.Cu") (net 5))
 (segment (start 147.3 99.866) (end 147.4 99.866) (width 0.2) (layer "F.Cu") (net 5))
 (segment (start 113.86 79.856) (end 112.58 78.576) (width 0.2) (layer "F.Cu") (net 5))
 (segment (start 164.46 134.406) (end 164.36 134.306) (width 0.2) (layer "F.Cu") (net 5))
 (segment (start 127.36 134.306) (end 127.96 134.306) (width 0.2) (layer "F.Cu") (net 5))
 (segment (start 142.86 117.306) (end 140.26 114.706) (width 0.2) (layer "F.Cu") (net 5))
 (segment (start 140.26 107.006) (end 147.4 99.866) (width 0.2) (layer "F.Cu") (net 5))
 (segment (start 130.36 117.306) (end 125.61 122.056) (width 0.2) (layer "F.Cu") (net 5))
 (segment (start 116.11 79.856) (end 121.36 85.106) (width 0.2) (layer "F.Cu") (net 5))
 (segment (start 127.36 148.306) (end 127.36 134.306) (width 0.2) (layer "F.Cu") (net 5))
 (segment (start 113.86 79.856) (end 140.26 106.256) (width 0.2) (layer "F.Cu") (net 5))
 (segment (start 172.76 84.326) (end 176.88 80.206) (width 0.2) (layer "F.Cu") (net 5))
 (segment (start 140.26 106.256) (end 140.26 107.006) (width 0.2) (layer "F.Cu") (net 5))
 (segment (start 113.86 79.856) (end 116.11 79.856) (width 0.2) (layer "F.Cu") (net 5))
 (segment (start 182.01 80.206) (end 182.61 80.806) (width 0.2) (layer "F.Cu") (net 5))
 (segment (start 164.56 134.306) (end 164.46 134.406) (width 0.2) (layer "F.Cu") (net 5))
 (segment (start 145.86 134.306) (end 127.36 134.306) (width 0.2) (layer "F.Cu") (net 5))
 (segment (start 182.61 131.556) (end 179.86 134.306) (width 0.2) (layer "F.Cu") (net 5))
 (segment (start 182.61 80.806) (end 182.61 131.556) (width 0.2) (layer "F.Cu") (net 5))
 (segment (start 130.36 151.306) (end 127.36 148.306) (width 0.2) (layer "F.Cu") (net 5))
 (segment (start 112.58 78.576) (end 112.58 67.606) (width 0.2) (layer "F.Cu") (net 5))
 (segment (start 147.36 99.246) (end 147.42 99.306) (width 0.2) (layer "F.Cu") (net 5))
 (segment (start 176.88 80.206) (end 182.01 80.206) (width 0.2) (layer "F.Cu") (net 5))
 (via (at 164.36 134.306) (size 0.6) (drill 0.3) (layers "F.Cu" "B.Cu") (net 5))
 (segment (start 164.36 134.306) (end 158.36 134.306) (width 0.2) (layer "B.Cu") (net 5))
 (segment (start 126.89 69.686) (end 128.36 68.216) (width 0.2) (layer "F.Cu") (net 16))
 (segment (start 126.89 72.606) (end 126.89 69.686) (width 0.2) (layer "F.Cu") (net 16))
 (segment (start 132.4035 72.606) (end 143.631 83.8335) (width 0.2) (layer "F.Cu") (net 1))
 (segment (start 145.3185 86.506) (end 149.5635 86.506) (width 0.2) (layer "F.Cu") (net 1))
 (segment (start 143.631 84.8185) (end 145.3185 86.506) (width 0.2) (layer "F.Cu") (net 1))
 (segment (start 160.86 108.316) (end 164.01 108.316) (width 0.2) (layer "F.Cu") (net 1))
 (segment (start 149.5635 86.506) (end 151.251 84.8185) (width 0.2) (layer "F.Cu") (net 1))
 (segment (start 167.16 108.316) (end 167.16 104.306) (width 0.2) (layer "F.Cu") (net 1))
 (segment (start 167.16 108.316) (end 164.01 108.316) (width 0.2) (layer "F.Cu") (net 1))
 (segment (start 128.16 72.606) (end 132.4035 72.606) (width 0.2) (layer "F.Cu") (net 1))
 (segment (start 143.631 83.8335) (end 143.631 84.8185) (width 0.2) (layer "F.Cu") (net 1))
 (segment (start 151.251 84.8185) (end 151.251 83.8335) (width 0.2) (layer "F.Cu") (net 1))
 (segment (start 157.56 104.006) (end 157.56 99.866) (width 0.2) (layer "F.Cu") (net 1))
 (segment (start 151.9475 83.137) (end 166.491 83.137) (width 0.2) (layer "F.Cu") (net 1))
 (segment (start 166.491 83.137) (end 167.68 84.326) (width 0.2) (layer "F.Cu") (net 1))
 (segment (start 160.86 108.316) (end 160.86 107.306) (width 0.2) (layer "F.Cu") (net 1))
 (segment (start 167.16 108.316) (end 170.31 108.316) (width 0.2) (layer "F.Cu") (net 1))
 (segment (start 160.86 107.306) (end 157.56 104.006) (width 0.2) (layer "F.Cu") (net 1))
 (segment (start 151.251 83.8335) (end 151.9475 83.137) (width 0.2) (layer "F.Cu") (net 1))
 (segment (start 170.31 108.316) (end 173.46 108.316) (width 0.2) (layer "F.Cu") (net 1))
 (via (at 167.16 104.306) (size 0.6) (drill 0.3) (layers "F.Cu" "B.Cu") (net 1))
 (segment (start 168.929 85.575) (end 167.68 84.326) (width 0.2) (layer "B.Cu") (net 1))
 (segment (start 167.16 104.306) (end 168.929 102.537) (width 0.2) (layer "B.Cu") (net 1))
 (segment (start 168.929 102.537) (end 168.929 85.575) (width 0.2) (layer "B.Cu") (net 1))
 (segment (start 156.331 65.195) (end 157.52 64.006) (width 0.2) (layer "F.Cu") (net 27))
 (segment (start 154.249 65.195) (end 156.331 65.195) (width 0.2) (layer "F.Cu") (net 27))
 (segment (start 129.46 50.206) (end 152.96 50.206) (width 0.2) (layer "F.Cu") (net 27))
 (segment (start 153.76 51.006) (end 153.76 64.706) (width 0.2) (layer "F.Cu") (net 27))
 (segment (start 128.36 51.306) (end 129.46 50.206) (width 0.2) (layer "F.Cu") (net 27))
 (segment (start 153.76 64.706) (end 154.249 65.195) (width 0.2) (layer "F.Cu") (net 27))
 (segment (start 152.96 50.206) (end 153.76 51.006) (width 0.2) (layer "F.Cu") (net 27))
 (segment (start 128.36 60.596) (end 128.36 51.306) (width 0.2) (layer "F.Cu") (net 27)))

